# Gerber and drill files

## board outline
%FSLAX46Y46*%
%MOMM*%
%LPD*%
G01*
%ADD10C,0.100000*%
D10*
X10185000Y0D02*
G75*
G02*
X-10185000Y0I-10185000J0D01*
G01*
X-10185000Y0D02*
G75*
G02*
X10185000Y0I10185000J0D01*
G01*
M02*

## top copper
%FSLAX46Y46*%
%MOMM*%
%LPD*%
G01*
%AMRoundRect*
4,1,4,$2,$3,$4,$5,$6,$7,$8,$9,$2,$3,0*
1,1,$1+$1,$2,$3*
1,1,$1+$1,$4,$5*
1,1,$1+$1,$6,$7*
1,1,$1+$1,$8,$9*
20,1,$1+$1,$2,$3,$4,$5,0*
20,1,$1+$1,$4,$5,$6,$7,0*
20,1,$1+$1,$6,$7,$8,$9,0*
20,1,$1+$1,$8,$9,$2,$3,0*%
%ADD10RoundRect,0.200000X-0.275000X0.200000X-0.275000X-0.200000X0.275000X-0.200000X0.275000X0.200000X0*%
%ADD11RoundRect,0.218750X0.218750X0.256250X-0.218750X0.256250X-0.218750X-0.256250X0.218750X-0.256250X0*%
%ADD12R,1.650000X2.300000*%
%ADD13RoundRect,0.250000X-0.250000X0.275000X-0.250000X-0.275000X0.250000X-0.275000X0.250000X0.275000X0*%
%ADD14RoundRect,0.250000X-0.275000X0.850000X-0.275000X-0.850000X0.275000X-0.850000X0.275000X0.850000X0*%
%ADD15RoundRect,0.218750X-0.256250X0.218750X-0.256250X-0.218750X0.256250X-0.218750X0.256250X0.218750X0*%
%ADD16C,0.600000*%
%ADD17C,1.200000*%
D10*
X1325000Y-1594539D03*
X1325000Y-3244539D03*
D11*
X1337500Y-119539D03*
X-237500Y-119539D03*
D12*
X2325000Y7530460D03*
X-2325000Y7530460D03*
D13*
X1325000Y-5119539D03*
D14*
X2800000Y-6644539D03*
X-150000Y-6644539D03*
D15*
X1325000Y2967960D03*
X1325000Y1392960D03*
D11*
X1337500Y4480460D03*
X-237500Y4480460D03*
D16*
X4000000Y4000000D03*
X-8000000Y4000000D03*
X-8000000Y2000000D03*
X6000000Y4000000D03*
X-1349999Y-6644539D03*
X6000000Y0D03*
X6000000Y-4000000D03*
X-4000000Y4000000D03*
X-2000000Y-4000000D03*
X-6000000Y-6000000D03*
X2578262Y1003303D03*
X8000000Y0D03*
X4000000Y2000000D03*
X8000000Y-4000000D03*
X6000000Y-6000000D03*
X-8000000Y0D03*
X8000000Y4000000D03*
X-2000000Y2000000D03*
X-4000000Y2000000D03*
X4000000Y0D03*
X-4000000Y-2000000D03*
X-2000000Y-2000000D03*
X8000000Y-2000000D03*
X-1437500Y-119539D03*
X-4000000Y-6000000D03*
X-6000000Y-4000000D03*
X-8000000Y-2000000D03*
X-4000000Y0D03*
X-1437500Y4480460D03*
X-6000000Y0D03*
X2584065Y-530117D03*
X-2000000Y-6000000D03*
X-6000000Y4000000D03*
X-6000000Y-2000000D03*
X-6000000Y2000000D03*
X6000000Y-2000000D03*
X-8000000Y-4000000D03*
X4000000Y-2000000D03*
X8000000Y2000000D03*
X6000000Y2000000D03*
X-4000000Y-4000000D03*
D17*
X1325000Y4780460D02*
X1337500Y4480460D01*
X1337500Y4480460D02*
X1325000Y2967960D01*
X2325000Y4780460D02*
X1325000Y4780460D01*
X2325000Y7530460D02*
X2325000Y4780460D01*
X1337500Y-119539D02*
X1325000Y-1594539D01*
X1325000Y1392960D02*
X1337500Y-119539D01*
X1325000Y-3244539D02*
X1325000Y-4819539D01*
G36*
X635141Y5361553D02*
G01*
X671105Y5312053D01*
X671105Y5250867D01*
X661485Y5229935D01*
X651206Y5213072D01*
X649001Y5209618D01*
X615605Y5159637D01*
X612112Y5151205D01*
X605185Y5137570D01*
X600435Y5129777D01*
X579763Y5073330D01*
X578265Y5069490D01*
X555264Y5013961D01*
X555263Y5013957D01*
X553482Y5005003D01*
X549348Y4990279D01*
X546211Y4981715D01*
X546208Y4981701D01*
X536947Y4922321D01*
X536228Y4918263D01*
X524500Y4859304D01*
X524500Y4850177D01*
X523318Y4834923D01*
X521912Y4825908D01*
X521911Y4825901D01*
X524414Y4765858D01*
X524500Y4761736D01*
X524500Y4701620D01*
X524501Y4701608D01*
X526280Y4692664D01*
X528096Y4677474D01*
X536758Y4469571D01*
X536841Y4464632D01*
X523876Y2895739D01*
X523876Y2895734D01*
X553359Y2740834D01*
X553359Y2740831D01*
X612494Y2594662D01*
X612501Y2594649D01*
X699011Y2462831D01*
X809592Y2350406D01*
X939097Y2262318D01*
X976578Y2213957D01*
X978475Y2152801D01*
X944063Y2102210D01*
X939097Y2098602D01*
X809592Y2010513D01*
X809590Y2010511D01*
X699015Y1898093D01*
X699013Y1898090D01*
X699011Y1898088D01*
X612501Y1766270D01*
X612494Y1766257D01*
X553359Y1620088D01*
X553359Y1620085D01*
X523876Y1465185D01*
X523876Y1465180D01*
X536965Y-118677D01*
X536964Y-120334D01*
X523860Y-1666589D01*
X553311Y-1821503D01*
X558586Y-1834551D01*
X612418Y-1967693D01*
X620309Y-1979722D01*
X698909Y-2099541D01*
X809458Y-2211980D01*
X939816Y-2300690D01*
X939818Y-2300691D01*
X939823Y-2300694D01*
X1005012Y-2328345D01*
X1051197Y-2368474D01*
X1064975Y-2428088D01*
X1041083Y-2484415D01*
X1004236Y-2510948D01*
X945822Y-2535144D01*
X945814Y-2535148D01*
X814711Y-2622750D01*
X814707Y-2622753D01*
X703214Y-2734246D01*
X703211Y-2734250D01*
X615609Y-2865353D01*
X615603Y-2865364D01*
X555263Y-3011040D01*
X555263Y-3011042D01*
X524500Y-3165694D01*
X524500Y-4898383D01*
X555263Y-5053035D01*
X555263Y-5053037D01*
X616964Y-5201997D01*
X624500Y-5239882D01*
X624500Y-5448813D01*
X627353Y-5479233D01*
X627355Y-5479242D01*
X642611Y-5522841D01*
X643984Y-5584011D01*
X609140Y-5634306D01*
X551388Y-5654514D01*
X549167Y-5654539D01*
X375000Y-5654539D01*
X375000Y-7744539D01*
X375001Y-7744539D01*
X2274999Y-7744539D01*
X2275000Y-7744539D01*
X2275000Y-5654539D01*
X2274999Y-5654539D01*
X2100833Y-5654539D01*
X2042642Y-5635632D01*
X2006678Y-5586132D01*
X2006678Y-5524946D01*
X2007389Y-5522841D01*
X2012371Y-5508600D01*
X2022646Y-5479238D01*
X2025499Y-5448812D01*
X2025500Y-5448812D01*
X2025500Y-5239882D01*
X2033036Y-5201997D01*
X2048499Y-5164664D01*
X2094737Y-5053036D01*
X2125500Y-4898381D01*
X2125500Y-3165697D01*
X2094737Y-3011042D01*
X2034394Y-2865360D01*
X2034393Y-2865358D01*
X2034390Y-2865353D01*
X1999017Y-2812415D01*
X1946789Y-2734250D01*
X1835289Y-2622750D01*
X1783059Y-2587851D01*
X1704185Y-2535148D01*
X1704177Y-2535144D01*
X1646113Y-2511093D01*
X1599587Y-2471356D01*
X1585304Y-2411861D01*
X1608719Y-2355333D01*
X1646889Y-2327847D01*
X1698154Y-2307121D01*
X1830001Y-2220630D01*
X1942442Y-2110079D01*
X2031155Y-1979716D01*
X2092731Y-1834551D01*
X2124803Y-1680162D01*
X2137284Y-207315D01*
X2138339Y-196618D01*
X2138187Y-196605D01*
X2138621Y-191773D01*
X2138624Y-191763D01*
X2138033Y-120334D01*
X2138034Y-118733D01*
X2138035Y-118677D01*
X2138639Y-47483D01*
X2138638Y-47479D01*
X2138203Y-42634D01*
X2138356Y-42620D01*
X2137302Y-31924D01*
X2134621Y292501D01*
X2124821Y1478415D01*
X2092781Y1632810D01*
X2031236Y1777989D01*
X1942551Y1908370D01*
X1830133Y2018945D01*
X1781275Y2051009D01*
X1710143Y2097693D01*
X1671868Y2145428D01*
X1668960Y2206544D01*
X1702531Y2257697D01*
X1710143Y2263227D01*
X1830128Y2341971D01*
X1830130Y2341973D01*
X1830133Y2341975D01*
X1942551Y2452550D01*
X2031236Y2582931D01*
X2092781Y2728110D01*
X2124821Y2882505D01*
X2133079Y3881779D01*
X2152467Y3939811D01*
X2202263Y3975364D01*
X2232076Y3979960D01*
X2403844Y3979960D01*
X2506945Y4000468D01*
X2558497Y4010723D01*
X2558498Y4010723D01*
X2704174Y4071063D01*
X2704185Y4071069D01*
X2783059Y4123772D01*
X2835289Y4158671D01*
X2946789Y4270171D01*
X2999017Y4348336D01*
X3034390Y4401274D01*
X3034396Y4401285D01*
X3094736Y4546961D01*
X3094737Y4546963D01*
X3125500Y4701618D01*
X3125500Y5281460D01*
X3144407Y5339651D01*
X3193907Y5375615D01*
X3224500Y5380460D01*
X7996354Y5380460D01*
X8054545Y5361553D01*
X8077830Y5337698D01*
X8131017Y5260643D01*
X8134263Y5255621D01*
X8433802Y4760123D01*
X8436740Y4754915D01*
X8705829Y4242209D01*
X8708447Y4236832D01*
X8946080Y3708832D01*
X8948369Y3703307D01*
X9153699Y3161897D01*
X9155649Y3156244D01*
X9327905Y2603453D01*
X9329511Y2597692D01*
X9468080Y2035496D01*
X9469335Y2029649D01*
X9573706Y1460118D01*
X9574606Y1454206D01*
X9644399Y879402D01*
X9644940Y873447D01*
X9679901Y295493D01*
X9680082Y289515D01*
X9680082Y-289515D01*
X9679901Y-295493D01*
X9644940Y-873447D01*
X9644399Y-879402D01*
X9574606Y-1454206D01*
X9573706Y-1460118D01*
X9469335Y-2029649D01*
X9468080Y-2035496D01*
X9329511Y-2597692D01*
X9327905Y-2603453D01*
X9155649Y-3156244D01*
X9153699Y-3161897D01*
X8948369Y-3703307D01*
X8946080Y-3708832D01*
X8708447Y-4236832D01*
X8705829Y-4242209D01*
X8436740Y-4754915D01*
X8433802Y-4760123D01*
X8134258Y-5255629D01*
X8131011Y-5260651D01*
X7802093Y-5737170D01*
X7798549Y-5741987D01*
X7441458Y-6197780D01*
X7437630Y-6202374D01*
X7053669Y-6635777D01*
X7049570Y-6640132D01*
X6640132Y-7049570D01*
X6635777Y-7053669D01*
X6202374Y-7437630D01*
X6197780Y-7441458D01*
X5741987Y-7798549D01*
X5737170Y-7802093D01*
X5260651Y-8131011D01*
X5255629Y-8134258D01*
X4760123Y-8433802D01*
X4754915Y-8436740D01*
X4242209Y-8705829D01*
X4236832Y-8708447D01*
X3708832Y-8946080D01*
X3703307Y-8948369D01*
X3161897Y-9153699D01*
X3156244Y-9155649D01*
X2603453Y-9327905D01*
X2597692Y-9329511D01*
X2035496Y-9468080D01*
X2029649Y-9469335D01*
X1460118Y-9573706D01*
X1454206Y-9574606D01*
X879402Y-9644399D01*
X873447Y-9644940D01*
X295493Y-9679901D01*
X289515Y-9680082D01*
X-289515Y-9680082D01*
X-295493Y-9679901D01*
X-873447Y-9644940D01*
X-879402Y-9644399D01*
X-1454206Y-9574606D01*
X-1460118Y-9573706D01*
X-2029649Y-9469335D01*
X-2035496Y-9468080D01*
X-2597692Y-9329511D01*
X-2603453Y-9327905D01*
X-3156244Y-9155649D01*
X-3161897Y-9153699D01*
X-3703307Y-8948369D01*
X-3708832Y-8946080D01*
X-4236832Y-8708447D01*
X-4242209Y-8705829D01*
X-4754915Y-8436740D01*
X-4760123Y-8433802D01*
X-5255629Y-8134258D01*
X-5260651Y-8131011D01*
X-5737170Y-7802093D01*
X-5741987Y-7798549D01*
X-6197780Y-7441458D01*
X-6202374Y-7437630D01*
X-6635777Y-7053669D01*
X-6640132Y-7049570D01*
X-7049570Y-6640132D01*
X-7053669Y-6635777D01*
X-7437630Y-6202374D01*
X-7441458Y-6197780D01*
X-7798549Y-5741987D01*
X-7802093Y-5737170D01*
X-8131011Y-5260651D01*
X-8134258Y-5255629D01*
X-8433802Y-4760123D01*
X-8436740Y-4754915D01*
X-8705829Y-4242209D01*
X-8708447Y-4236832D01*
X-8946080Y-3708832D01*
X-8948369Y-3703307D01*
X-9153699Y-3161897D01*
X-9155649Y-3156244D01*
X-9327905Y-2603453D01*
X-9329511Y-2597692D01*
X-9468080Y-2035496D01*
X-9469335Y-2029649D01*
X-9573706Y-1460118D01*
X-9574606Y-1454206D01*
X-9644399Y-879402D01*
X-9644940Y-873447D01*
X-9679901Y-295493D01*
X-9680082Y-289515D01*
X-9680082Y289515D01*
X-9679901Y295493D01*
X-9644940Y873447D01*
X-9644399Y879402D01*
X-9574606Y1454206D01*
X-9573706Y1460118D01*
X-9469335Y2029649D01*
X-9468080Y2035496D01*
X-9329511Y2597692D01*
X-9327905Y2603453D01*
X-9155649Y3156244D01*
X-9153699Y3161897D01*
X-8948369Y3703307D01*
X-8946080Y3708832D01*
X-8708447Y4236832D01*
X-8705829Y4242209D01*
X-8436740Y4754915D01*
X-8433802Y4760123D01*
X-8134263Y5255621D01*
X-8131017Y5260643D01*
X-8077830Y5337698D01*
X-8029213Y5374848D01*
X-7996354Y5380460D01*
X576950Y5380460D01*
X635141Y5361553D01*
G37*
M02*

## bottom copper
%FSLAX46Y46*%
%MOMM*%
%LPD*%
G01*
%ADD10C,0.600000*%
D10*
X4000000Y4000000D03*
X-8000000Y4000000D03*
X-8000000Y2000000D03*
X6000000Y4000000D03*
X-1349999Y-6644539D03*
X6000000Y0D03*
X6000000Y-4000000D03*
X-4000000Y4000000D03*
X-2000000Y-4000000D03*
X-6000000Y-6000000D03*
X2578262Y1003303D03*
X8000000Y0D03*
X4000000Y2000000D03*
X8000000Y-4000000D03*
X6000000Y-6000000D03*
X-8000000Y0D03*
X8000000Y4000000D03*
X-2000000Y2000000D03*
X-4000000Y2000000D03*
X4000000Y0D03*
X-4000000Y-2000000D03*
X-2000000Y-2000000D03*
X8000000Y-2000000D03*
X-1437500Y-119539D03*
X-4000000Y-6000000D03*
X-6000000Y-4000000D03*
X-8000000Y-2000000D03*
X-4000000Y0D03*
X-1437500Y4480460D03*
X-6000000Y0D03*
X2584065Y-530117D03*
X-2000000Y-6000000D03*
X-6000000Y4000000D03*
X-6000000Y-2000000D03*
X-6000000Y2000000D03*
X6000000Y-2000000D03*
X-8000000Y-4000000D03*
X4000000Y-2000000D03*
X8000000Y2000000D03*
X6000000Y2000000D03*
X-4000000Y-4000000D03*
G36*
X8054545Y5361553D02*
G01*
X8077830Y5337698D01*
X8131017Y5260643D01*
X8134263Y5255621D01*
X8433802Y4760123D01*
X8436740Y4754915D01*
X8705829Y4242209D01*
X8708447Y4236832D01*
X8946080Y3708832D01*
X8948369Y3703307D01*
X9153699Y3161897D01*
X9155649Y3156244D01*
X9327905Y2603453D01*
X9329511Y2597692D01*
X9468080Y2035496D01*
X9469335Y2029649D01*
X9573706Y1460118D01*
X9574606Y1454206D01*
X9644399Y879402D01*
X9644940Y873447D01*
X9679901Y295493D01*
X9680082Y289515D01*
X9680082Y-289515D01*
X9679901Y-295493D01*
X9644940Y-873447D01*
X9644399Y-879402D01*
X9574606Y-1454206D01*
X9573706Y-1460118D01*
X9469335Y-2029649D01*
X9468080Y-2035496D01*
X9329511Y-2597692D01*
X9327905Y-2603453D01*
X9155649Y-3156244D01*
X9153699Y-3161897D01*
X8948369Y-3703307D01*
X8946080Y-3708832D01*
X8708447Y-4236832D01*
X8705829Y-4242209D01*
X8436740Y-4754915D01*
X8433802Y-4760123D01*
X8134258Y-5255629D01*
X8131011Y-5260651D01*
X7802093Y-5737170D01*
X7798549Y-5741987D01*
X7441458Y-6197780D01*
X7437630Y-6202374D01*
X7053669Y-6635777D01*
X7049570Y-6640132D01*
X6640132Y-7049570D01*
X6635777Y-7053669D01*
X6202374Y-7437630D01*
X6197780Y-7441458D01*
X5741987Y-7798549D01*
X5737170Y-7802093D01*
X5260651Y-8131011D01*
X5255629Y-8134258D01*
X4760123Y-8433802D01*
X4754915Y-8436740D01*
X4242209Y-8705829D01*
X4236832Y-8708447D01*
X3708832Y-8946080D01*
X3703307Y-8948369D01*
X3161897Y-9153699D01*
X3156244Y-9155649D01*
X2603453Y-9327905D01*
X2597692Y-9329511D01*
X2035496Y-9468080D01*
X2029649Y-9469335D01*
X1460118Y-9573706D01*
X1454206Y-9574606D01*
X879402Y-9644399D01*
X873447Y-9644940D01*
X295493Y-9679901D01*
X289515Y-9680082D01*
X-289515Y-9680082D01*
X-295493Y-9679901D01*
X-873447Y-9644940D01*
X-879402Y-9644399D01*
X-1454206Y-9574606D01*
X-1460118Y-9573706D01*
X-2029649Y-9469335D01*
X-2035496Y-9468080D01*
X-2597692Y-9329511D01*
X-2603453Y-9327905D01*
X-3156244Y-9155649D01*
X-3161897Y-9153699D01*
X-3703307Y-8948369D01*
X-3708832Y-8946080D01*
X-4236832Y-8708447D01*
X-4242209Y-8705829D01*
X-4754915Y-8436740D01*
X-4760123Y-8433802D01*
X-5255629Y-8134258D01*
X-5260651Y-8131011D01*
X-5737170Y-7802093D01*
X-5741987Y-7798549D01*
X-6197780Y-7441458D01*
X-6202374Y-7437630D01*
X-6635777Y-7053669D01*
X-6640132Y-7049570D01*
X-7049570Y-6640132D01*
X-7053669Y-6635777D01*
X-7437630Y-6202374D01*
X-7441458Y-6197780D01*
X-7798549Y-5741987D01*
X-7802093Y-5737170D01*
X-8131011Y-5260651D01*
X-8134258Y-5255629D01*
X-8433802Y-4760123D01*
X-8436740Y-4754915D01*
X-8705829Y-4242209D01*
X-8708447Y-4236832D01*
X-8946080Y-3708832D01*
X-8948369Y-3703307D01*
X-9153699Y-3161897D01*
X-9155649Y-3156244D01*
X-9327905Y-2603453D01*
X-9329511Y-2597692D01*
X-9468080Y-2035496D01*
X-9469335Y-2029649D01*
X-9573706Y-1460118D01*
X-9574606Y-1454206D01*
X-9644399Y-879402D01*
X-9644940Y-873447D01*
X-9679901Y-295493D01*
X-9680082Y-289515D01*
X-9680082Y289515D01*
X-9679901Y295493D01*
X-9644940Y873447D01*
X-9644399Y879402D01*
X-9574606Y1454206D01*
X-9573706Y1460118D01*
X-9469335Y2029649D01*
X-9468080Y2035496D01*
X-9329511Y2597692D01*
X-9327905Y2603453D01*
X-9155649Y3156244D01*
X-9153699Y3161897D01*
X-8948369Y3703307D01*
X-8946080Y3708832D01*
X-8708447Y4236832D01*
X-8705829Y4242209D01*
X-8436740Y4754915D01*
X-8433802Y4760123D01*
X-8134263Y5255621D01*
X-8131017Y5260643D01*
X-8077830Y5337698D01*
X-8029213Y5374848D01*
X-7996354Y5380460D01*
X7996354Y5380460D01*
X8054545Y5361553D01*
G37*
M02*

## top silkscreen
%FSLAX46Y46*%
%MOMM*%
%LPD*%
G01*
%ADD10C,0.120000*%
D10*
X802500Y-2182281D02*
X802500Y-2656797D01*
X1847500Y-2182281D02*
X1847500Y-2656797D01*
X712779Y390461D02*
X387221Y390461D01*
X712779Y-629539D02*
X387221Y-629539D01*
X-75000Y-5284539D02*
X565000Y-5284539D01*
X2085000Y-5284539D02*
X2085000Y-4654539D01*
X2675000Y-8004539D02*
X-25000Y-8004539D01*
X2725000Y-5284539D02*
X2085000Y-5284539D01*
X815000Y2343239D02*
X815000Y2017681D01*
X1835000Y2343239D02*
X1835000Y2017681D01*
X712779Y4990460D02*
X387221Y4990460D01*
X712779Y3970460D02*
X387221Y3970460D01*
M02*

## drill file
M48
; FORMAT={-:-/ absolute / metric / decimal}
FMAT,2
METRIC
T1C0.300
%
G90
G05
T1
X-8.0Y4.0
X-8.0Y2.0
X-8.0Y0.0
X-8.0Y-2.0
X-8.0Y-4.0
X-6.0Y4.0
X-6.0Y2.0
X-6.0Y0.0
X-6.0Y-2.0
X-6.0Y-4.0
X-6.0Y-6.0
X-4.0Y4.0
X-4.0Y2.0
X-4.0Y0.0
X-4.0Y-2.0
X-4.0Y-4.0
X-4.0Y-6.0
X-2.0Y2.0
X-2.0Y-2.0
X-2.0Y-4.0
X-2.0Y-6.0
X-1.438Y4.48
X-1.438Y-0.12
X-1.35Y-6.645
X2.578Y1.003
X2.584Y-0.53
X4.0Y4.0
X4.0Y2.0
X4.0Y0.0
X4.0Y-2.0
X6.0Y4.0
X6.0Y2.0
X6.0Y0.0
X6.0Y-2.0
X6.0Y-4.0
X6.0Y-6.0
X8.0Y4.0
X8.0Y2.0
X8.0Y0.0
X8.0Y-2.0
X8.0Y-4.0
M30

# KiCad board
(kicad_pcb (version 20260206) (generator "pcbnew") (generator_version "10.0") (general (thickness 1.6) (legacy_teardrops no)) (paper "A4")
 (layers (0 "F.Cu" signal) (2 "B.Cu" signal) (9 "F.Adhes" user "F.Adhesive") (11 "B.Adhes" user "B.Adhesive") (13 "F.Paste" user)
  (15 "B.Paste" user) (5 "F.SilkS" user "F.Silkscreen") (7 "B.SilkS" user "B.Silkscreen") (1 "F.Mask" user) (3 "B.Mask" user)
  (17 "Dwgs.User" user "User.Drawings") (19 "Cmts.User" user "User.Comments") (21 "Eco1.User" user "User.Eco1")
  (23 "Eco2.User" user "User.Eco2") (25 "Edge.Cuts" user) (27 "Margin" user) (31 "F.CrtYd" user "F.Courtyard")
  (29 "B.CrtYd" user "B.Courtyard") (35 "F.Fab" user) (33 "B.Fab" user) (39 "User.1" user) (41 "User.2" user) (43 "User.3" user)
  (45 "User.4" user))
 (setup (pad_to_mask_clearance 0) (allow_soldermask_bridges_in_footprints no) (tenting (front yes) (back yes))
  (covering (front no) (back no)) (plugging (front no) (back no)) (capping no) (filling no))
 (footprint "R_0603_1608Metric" (layer "F.Cu") (at 1.325 2.419539 -90)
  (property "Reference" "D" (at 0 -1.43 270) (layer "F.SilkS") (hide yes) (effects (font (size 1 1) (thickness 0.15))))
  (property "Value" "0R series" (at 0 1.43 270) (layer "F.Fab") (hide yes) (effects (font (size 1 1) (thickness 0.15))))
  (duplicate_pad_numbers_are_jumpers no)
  (fp_line (start -0.237258 0.5225) (end 0.237258 0.5225) (stroke (width 0.12) (type solid)) (layer "F.SilkS"))
  (fp_line (start -0.237258 -0.5225) (end 0.237258 -0.5225) (stroke (width 0.12) (type solid)) (layer "F.SilkS"))
  (pad "1" smd roundrect (at -0.825 0 270) (size 0.8 0.95) (layers "F.Cu" "F.Mask" "F.Paste") (roundrect_rratio 0.25) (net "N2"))
  (pad "2" smd roundrect (at 0.825 0 270) (size 0.8 0.95) (layers "F.Cu" "F.Mask" "F.Paste") (roundrect_rratio 0.25) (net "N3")))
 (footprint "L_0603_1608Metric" (layer "F.Cu") (at 0.55 0.119539 180)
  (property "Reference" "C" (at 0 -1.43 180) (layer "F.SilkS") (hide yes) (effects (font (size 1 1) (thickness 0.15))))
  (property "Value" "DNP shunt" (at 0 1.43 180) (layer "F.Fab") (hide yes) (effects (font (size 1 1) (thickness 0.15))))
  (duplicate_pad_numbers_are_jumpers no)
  (fp_line (start -0.162779 0.51) (end 0.162779 0.51) (stroke (width 0.12) (type solid)) (layer "F.SilkS"))
  (fp_line (start -0.162779 -0.51) (end 0.162779 -0.51) (stroke (width 0.12) (type solid)) (layer "F.SilkS"))
  (pad "1" smd roundrect (at -0.7875 0 180) (size 0.875 0.95) (layers "F.Cu" "F.Mask" "F.Paste") (roundrect_rratio 0.25) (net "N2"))
  (pad "2" smd roundrect (at 0.7875 0 180) (size 0.875 0.95) (layers "F.Cu" "F.Mask" "F.Paste") (roundrect_rratio 0.25) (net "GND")))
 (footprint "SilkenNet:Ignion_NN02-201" (layer "F.Cu") (at 0 -7.53046)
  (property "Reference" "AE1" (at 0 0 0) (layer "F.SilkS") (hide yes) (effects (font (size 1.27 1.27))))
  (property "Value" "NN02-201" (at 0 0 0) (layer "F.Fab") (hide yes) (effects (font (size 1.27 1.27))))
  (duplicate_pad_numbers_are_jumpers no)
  (pad "1" smd rect (at 2.325 0) (size 1.65 2.3) (layers "F.Cu" "F.Mask" "F.Paste") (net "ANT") (thermal_bridge_angle 45))
  (pad "2" smd rect (at -2.325 0) (size 1.65 2.3) (layers "F.Cu" "F.Mask" "F.Paste") (thermal_bridge_angle 45)))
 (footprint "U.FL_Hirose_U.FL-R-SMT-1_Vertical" (layer "F.Cu") (at 1.325 6.644539 -90)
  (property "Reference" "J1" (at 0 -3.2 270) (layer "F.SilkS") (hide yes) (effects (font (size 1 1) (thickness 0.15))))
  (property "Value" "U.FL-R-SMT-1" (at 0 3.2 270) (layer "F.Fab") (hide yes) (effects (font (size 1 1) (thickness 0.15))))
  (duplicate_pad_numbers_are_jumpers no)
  (fp_line (start -1.36 1.4) (end -1.36 0.76) (stroke (width 0.12) (type solid)) (layer "F.SilkS"))
  (fp_line (start -1.36 -0.76) (end -1.99 -0.76) (stroke (width 0.12) (type solid)) (layer "F.SilkS"))
  (fp_line (start 1.36 -1.35) (end 1.36 1.35) (stroke (width 0.12) (type solid)) (layer "F.SilkS"))
  (fp_line (start -1.36 -1.4) (end -1.36 -0.76) (stroke (width 0.12) (type solid)) (layer "F.SilkS"))
  (pad "1" smd roundrect (at -1.525 0 270) (size 1.05 1) (layers "F.Cu" "F.Mask" "F.Paste") (roundrect_rratio 0.25) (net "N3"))
  (pad "2" smd roundrect (at 0 -1.475 270) (size 2.2 1.05) (layers "F.Cu" "F.Mask" "F.Paste") (roundrect_rratio 0.2380952381) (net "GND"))
  (pad "2" smd roundrect (at 0 1.475 270) (size 2.2 1.05) (layers "F.Cu" "F.Mask" "F.Paste") (roundrect_rratio 0.2380952381) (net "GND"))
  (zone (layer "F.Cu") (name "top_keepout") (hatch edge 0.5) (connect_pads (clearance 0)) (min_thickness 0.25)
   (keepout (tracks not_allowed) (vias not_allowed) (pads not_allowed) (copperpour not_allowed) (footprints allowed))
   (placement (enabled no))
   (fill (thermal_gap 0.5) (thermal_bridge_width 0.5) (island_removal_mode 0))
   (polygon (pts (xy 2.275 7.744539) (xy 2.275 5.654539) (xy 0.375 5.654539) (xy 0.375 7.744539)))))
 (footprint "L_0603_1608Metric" (layer "F.Cu") (at 1.325 -2.18046 -90)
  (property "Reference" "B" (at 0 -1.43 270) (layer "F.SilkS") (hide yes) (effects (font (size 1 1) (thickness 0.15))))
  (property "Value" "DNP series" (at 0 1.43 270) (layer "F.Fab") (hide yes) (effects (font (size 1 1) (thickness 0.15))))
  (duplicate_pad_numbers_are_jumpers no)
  (fp_line (start -0.162779 0.51) (end 0.162779 0.51) (stroke (width 0.12) (type solid)) (layer "F.SilkS"))
  (fp_line (start -0.162779 -0.51) (end 0.162779 -0.51) (stroke (width 0.12) (type solid)) (layer "F.SilkS"))
  (pad "1" smd roundrect (at -0.7875 0 270) (size 0.875 0.95) (layers "F.Cu" "F.Mask" "F.Paste") (roundrect_rratio 0.25) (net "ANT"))
  (pad "2" smd roundrect (at 0.7875 0 270) (size 0.875 0.95) (layers "F.Cu" "F.Mask" "F.Paste") (roundrect_rratio 0.25) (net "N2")))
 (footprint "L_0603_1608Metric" (layer "F.Cu") (at 0.55 -4.48046 180)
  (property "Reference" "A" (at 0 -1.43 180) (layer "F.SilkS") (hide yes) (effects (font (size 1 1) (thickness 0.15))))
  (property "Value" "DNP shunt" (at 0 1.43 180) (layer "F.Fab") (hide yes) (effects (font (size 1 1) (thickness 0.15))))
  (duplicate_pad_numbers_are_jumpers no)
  (fp_line (start -0.162779 0.51) (end 0.162779 0.51) (stroke (width 0.12) (type solid)) (layer "F.SilkS"))
  (fp_line (start -0.162779 -0.51) (end 0.162779 -0.51) (stroke (width 0.12) (type solid)) (layer "F.SilkS"))
  (pad "1" smd roundrect (at -0.7875 0 180) (size 0.875 0.95) (layers "F.Cu" "F.Mask" "F.Paste") (roundrect_rratio 0.25) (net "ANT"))
  (pad "2" smd roundrect (at 0.7875 0 180) (size 0.875 0.95) (layers "F.Cu" "F.Mask" "F.Paste") (roundrect_rratio 0.25) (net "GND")))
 (gr_circle (center 0 0) (end 10.185 0) (stroke (width 0.1) (type default)) (fill no) (layer "Edge.Cuts"))
 (via (at 4 -4) (size 0.6) (drill 0.3) (layers "F.Cu" "B.Cu") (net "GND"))
 (via (at -8 -4) (size 0.6) (drill 0.3) (layers "F.Cu" "B.Cu") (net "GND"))
 (via (at -8 -2) (size 0.6) (drill 0.3) (layers "F.Cu" "B.Cu") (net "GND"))
 (via (at 6 -4) (size 0.6) (drill 0.3) (layers "F.Cu" "B.Cu") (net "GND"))
 (via (at -1.349999 6.644539) (size 0.6) (drill 0.3) (layers "F.Cu" "B.Cu") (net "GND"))
 (via (at 6 0) (size 0.6) (drill 0.3) (layers "F.Cu" "B.Cu") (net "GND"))
 (via (at 6 4) (size 0.6) (drill 0.3) (layers "F.Cu" "B.Cu") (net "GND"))
 (via (at -4 -4) (size 0.6) (drill 0.3) (layers "F.Cu" "B.Cu") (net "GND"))
 (via (at -2 4) (size 0.6) (drill 0.3) (layers "F.Cu" "B.Cu") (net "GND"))
 (via (at -6 6) (size 0.6) (drill 0.3) (layers "F.Cu" "B.Cu") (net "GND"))
 (via (at 2.578262 -1.003303) (size 0.6) (drill 0.3) (layers "F.Cu" "B.Cu") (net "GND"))
 (via (at 8 0) (size 0.6) (drill 0.3) (layers "F.Cu" "B.Cu") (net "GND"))
 (via (at 4 -2) (size 0.6) (drill 0.3) (layers "F.Cu" "B.Cu") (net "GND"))
 (via (at 8 4) (size 0.6) (drill 0.3) (layers "F.Cu" "B.Cu") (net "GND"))
 (via (at 6 6) (size 0.6) (drill 0.3) (layers "F.Cu" "B.Cu") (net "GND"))
 (via (at -8 0) (size 0.6) (drill 0.3) (layers "F.Cu" "B.Cu") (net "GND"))
 (via (at 8 -4) (size 0.6) (drill 0.3) (layers "F.Cu" "B.Cu") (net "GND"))
 (via (at -2 -2) (size 0.6) (drill 0.3) (layers "F.Cu" "B.Cu") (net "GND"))
 (via (at -4 -2) (size 0.6) (drill 0.3) (layers "F.Cu" "B.Cu") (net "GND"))
 (via (at 4 0) (size 0.6) (drill 0.3) (layers "F.Cu" "B.Cu") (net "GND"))
 (via (at -4 2) (size 0.6) (drill 0.3) (layers "F.Cu" "B.Cu") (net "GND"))
 (via (at -2 2) (size 0.6) (drill 0.3) (layers "F.Cu" "B.Cu") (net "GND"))
 (via (at 8 2) (size 0.6) (drill 0.3) (layers "F.Cu" "B.Cu") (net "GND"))
 (via (at -1.4375 0.119539) (size 0.6) (drill 0.3) (layers "F.Cu" "B.Cu") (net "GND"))
 (via (at -4 6) (size 0.6) (drill 0.3) (layers "F.Cu" "B.Cu") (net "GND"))
 (via (at -6 4) (size 0.6) (drill 0.3) (layers "F.Cu" "B.Cu") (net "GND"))
 (via (at -8 2) (size 0.6) (drill 0.3) (layers "F.Cu" "B.Cu") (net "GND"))
 (via (at -4 0) (size 0.6) (drill 0.3) (layers "F.Cu" "B.Cu") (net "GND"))
 (via (at -1.4375 -4.48046) (size 0.6) (drill 0.3) (layers "F.Cu" "B.Cu") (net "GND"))
 (via (at -6 0) (size 0.6) (drill 0.3) (layers "F.Cu" "B.Cu") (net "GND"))
 (via (at 2.584065 0.530117) (size 0.6) (drill 0.3) (layers "F.Cu" "B.Cu") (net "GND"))
 (via (at -2 6) (size 0.6) (drill 0.3) (layers "F.Cu" "B.Cu") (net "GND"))
 (via (at -6 -4) (size 0.6) (drill 0.3) (layers "F.Cu" "B.Cu") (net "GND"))
 (via (at -6 2) (size 0.6) (drill 0.3) (layers "F.Cu" "B.Cu") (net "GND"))
 (via (at -6 -2) (size 0.6) (drill 0.3) (layers "F.Cu" "B.Cu") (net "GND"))
 (via (at 6 2) (size 0.6) (drill 0.3) (layers "F.Cu" "B.Cu") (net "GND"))
 (via (at -8 4) (size 0.6) (drill 0.3) (layers "F.Cu" "B.Cu") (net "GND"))
 (via (at 4 2) (size 0.6) (drill 0.3) (layers "F.Cu" "B.Cu") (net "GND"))
 (via (at 8 -2) (size 0.6) (drill 0.3) (layers "F.Cu" "B.Cu") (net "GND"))
 (via (at 6 -2) (size 0.6) (drill 0.3) (layers "F.Cu" "B.Cu") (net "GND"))
 (via (at -4 4) (size 0.6) (drill 0.3) (layers "F.Cu" "B.Cu") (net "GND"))
 (segment (start 1.325 -4.78046) (end 1.3375 -4.48046) (width 1.2) (layer "F.Cu") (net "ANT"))
 (segment (start 1.3375 -4.48046) (end 1.325 -2.96796) (width 1.2) (layer "F.Cu") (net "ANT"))
 (segment (start 2.325 -4.78046) (end 1.325 -4.78046) (width 1.2) (layer "F.Cu") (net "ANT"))
 (segment (start 2.325 -7.53046) (end 2.325 -4.78046) (width 1.2) (layer "F.Cu") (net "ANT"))
 (segment (start 1.3375 0.119539) (end 1.325 1.594539) (width 1.2) (layer "F.Cu") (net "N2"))
 (segment (start 1.325 -1.39296) (end 1.3375 0.119539) (width 1.2) (layer "F.Cu") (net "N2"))
 (segment (start 1.325 3.244539) (end 1.325 4.819539) (width 1.2) (layer "F.Cu") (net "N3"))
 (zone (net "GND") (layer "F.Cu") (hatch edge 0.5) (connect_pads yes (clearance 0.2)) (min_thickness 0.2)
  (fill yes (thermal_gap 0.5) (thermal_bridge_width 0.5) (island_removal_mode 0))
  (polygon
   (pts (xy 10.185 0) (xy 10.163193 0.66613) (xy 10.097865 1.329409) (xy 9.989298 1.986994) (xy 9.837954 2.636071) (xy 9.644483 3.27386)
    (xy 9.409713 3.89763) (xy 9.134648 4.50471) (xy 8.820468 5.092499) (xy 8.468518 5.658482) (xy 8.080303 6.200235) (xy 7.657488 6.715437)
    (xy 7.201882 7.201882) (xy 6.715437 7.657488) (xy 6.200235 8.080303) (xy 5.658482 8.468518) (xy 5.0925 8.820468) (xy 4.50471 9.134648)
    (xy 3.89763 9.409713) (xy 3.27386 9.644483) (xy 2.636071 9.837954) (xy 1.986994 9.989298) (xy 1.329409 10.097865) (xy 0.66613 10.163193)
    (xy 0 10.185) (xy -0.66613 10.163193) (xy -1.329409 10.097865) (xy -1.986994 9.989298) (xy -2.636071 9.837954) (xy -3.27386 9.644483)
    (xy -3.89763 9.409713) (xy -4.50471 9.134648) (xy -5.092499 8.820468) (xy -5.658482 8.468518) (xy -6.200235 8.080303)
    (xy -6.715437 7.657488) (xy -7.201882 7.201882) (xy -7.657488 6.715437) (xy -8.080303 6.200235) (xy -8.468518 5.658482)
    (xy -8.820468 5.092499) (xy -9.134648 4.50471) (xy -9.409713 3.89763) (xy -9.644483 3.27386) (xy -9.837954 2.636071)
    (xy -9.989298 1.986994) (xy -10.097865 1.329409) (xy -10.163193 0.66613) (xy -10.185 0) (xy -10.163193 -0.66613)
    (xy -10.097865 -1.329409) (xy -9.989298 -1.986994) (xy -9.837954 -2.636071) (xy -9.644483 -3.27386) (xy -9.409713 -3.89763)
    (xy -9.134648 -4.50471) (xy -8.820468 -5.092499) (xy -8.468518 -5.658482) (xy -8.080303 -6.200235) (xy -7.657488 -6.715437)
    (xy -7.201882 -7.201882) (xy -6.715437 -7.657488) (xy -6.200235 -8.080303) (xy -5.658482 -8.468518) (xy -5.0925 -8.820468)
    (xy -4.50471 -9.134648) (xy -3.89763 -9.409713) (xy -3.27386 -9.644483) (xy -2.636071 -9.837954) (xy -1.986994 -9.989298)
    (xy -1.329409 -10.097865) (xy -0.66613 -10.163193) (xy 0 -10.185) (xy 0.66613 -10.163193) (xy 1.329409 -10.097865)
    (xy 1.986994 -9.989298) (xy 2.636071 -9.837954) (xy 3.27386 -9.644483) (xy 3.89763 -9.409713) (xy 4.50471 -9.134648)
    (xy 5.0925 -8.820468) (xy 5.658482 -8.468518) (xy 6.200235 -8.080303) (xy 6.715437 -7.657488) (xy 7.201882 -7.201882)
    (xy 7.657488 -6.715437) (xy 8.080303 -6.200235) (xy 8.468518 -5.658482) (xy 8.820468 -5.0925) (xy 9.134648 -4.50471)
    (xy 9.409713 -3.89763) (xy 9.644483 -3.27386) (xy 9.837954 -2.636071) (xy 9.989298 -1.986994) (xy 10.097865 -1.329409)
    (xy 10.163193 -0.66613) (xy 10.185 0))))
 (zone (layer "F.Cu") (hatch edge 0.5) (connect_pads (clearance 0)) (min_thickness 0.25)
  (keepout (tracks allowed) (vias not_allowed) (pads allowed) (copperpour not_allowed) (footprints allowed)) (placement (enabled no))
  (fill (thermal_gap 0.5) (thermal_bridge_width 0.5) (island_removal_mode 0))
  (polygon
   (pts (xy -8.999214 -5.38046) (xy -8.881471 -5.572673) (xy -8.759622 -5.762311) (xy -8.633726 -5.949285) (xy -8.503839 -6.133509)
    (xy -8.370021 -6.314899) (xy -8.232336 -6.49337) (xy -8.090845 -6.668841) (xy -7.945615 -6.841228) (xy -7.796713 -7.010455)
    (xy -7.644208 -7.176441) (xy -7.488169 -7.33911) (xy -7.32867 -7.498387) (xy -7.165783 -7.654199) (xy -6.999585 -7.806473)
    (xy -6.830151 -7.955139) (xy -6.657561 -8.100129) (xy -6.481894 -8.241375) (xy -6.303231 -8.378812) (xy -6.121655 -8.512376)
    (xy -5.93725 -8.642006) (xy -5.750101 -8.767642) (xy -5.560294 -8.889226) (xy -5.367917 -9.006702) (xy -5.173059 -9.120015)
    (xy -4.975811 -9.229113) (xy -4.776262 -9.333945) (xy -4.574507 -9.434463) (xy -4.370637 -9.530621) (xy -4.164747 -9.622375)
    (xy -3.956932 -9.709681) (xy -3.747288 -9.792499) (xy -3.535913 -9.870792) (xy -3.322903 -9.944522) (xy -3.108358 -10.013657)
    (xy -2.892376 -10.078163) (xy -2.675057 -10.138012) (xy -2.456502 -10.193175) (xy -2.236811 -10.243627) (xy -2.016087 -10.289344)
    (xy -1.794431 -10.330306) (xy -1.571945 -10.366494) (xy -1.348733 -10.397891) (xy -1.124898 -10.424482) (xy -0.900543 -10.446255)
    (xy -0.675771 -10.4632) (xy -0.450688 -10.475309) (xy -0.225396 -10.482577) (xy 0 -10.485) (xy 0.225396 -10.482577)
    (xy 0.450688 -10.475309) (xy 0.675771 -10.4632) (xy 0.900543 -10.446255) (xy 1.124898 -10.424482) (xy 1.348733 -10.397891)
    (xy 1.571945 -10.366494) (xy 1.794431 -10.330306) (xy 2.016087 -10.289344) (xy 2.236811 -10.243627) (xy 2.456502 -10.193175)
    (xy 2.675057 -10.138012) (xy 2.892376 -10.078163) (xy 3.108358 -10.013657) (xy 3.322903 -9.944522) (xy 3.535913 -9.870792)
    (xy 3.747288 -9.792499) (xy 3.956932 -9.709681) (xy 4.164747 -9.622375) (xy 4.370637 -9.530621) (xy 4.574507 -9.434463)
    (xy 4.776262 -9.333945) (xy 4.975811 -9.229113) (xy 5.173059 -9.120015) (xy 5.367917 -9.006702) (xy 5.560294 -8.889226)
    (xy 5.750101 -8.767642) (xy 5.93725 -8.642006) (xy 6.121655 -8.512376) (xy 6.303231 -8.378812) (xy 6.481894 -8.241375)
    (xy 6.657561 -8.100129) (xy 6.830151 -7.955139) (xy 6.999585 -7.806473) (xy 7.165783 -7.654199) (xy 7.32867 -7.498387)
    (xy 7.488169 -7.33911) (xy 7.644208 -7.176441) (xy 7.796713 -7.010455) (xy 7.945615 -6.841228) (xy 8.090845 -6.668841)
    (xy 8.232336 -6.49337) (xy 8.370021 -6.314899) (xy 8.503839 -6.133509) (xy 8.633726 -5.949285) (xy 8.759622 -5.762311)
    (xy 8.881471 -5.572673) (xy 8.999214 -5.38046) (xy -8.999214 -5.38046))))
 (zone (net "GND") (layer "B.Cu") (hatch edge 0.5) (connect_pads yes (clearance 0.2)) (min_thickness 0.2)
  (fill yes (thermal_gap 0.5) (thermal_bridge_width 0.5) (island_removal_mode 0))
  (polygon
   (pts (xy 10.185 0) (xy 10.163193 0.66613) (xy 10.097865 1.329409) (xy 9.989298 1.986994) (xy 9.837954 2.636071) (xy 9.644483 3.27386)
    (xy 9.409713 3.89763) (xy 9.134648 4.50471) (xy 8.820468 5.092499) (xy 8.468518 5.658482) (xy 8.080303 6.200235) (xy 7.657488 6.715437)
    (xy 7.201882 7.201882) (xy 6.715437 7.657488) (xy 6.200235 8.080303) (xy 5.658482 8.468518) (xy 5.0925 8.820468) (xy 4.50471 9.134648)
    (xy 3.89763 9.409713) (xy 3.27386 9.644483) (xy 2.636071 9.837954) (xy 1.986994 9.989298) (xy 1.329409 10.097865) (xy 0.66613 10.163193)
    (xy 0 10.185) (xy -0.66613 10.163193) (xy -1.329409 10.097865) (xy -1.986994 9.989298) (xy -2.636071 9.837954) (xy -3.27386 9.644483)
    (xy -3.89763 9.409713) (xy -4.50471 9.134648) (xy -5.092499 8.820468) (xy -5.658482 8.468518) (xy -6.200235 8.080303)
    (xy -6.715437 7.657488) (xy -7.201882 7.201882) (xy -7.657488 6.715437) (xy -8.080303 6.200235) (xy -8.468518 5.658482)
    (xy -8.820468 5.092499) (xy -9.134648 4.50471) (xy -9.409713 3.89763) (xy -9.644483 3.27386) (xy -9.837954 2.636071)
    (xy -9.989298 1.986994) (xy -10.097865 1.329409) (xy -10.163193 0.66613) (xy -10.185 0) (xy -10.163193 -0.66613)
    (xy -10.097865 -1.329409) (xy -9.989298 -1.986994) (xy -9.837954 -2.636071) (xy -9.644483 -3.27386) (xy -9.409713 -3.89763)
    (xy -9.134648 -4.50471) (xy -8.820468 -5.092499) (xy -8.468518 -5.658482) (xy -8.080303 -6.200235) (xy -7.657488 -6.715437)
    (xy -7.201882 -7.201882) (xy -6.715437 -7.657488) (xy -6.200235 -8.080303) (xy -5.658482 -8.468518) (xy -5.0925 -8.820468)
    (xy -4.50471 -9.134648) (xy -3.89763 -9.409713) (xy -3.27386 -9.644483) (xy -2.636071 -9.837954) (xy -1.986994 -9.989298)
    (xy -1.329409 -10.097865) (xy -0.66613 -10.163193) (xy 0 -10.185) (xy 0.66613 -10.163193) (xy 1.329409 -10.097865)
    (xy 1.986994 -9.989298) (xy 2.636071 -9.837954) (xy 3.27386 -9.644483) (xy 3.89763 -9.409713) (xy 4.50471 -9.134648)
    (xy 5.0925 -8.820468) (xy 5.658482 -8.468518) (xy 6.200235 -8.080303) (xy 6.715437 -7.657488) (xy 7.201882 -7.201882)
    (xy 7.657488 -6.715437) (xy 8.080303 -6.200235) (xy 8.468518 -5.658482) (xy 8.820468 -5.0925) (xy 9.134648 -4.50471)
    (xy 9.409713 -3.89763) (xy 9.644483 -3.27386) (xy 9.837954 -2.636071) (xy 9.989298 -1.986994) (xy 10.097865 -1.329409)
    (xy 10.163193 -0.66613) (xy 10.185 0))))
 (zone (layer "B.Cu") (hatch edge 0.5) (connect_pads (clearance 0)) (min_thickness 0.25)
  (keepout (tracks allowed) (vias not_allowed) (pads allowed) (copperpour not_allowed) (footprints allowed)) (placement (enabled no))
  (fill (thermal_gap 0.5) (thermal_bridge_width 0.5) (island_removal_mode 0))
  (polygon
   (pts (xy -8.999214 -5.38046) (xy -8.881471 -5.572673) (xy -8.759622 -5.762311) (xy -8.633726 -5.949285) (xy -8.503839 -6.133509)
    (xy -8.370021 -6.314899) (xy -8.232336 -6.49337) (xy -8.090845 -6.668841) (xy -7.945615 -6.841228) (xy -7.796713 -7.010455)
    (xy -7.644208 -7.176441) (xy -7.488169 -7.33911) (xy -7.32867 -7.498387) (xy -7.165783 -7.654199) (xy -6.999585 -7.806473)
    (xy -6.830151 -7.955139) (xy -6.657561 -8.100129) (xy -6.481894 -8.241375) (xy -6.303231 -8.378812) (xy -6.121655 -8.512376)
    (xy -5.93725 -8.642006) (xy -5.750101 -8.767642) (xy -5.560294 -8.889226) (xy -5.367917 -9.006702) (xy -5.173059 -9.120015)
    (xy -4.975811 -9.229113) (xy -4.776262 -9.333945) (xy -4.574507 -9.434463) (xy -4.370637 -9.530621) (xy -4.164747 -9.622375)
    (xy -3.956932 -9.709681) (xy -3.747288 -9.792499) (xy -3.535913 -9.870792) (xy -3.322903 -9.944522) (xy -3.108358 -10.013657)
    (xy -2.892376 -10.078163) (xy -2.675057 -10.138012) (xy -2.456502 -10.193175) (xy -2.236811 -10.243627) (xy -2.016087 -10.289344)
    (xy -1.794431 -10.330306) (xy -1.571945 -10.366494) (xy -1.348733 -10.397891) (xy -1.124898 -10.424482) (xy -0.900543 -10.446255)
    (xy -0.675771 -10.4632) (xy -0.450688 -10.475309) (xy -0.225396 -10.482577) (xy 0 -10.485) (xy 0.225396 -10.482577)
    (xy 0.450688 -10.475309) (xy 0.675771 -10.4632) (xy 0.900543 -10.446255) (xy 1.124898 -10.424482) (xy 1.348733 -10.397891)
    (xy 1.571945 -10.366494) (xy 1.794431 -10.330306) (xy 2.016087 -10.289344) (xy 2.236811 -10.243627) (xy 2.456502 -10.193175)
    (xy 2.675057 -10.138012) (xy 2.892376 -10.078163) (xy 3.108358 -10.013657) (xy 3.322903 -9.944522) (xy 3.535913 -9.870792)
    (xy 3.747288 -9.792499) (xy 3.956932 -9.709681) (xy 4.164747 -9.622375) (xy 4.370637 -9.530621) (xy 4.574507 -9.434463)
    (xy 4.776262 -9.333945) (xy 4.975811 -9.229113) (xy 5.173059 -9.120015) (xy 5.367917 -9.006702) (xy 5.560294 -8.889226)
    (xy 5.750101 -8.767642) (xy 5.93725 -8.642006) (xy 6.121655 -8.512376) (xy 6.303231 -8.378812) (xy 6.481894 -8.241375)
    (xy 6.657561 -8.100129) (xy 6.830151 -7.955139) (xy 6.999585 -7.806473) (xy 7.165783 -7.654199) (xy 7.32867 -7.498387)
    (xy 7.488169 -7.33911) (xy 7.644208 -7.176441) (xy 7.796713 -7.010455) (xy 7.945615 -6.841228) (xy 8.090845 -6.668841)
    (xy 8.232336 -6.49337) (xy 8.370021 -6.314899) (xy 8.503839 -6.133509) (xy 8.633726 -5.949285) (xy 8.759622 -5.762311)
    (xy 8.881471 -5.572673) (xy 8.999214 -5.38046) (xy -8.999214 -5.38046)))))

